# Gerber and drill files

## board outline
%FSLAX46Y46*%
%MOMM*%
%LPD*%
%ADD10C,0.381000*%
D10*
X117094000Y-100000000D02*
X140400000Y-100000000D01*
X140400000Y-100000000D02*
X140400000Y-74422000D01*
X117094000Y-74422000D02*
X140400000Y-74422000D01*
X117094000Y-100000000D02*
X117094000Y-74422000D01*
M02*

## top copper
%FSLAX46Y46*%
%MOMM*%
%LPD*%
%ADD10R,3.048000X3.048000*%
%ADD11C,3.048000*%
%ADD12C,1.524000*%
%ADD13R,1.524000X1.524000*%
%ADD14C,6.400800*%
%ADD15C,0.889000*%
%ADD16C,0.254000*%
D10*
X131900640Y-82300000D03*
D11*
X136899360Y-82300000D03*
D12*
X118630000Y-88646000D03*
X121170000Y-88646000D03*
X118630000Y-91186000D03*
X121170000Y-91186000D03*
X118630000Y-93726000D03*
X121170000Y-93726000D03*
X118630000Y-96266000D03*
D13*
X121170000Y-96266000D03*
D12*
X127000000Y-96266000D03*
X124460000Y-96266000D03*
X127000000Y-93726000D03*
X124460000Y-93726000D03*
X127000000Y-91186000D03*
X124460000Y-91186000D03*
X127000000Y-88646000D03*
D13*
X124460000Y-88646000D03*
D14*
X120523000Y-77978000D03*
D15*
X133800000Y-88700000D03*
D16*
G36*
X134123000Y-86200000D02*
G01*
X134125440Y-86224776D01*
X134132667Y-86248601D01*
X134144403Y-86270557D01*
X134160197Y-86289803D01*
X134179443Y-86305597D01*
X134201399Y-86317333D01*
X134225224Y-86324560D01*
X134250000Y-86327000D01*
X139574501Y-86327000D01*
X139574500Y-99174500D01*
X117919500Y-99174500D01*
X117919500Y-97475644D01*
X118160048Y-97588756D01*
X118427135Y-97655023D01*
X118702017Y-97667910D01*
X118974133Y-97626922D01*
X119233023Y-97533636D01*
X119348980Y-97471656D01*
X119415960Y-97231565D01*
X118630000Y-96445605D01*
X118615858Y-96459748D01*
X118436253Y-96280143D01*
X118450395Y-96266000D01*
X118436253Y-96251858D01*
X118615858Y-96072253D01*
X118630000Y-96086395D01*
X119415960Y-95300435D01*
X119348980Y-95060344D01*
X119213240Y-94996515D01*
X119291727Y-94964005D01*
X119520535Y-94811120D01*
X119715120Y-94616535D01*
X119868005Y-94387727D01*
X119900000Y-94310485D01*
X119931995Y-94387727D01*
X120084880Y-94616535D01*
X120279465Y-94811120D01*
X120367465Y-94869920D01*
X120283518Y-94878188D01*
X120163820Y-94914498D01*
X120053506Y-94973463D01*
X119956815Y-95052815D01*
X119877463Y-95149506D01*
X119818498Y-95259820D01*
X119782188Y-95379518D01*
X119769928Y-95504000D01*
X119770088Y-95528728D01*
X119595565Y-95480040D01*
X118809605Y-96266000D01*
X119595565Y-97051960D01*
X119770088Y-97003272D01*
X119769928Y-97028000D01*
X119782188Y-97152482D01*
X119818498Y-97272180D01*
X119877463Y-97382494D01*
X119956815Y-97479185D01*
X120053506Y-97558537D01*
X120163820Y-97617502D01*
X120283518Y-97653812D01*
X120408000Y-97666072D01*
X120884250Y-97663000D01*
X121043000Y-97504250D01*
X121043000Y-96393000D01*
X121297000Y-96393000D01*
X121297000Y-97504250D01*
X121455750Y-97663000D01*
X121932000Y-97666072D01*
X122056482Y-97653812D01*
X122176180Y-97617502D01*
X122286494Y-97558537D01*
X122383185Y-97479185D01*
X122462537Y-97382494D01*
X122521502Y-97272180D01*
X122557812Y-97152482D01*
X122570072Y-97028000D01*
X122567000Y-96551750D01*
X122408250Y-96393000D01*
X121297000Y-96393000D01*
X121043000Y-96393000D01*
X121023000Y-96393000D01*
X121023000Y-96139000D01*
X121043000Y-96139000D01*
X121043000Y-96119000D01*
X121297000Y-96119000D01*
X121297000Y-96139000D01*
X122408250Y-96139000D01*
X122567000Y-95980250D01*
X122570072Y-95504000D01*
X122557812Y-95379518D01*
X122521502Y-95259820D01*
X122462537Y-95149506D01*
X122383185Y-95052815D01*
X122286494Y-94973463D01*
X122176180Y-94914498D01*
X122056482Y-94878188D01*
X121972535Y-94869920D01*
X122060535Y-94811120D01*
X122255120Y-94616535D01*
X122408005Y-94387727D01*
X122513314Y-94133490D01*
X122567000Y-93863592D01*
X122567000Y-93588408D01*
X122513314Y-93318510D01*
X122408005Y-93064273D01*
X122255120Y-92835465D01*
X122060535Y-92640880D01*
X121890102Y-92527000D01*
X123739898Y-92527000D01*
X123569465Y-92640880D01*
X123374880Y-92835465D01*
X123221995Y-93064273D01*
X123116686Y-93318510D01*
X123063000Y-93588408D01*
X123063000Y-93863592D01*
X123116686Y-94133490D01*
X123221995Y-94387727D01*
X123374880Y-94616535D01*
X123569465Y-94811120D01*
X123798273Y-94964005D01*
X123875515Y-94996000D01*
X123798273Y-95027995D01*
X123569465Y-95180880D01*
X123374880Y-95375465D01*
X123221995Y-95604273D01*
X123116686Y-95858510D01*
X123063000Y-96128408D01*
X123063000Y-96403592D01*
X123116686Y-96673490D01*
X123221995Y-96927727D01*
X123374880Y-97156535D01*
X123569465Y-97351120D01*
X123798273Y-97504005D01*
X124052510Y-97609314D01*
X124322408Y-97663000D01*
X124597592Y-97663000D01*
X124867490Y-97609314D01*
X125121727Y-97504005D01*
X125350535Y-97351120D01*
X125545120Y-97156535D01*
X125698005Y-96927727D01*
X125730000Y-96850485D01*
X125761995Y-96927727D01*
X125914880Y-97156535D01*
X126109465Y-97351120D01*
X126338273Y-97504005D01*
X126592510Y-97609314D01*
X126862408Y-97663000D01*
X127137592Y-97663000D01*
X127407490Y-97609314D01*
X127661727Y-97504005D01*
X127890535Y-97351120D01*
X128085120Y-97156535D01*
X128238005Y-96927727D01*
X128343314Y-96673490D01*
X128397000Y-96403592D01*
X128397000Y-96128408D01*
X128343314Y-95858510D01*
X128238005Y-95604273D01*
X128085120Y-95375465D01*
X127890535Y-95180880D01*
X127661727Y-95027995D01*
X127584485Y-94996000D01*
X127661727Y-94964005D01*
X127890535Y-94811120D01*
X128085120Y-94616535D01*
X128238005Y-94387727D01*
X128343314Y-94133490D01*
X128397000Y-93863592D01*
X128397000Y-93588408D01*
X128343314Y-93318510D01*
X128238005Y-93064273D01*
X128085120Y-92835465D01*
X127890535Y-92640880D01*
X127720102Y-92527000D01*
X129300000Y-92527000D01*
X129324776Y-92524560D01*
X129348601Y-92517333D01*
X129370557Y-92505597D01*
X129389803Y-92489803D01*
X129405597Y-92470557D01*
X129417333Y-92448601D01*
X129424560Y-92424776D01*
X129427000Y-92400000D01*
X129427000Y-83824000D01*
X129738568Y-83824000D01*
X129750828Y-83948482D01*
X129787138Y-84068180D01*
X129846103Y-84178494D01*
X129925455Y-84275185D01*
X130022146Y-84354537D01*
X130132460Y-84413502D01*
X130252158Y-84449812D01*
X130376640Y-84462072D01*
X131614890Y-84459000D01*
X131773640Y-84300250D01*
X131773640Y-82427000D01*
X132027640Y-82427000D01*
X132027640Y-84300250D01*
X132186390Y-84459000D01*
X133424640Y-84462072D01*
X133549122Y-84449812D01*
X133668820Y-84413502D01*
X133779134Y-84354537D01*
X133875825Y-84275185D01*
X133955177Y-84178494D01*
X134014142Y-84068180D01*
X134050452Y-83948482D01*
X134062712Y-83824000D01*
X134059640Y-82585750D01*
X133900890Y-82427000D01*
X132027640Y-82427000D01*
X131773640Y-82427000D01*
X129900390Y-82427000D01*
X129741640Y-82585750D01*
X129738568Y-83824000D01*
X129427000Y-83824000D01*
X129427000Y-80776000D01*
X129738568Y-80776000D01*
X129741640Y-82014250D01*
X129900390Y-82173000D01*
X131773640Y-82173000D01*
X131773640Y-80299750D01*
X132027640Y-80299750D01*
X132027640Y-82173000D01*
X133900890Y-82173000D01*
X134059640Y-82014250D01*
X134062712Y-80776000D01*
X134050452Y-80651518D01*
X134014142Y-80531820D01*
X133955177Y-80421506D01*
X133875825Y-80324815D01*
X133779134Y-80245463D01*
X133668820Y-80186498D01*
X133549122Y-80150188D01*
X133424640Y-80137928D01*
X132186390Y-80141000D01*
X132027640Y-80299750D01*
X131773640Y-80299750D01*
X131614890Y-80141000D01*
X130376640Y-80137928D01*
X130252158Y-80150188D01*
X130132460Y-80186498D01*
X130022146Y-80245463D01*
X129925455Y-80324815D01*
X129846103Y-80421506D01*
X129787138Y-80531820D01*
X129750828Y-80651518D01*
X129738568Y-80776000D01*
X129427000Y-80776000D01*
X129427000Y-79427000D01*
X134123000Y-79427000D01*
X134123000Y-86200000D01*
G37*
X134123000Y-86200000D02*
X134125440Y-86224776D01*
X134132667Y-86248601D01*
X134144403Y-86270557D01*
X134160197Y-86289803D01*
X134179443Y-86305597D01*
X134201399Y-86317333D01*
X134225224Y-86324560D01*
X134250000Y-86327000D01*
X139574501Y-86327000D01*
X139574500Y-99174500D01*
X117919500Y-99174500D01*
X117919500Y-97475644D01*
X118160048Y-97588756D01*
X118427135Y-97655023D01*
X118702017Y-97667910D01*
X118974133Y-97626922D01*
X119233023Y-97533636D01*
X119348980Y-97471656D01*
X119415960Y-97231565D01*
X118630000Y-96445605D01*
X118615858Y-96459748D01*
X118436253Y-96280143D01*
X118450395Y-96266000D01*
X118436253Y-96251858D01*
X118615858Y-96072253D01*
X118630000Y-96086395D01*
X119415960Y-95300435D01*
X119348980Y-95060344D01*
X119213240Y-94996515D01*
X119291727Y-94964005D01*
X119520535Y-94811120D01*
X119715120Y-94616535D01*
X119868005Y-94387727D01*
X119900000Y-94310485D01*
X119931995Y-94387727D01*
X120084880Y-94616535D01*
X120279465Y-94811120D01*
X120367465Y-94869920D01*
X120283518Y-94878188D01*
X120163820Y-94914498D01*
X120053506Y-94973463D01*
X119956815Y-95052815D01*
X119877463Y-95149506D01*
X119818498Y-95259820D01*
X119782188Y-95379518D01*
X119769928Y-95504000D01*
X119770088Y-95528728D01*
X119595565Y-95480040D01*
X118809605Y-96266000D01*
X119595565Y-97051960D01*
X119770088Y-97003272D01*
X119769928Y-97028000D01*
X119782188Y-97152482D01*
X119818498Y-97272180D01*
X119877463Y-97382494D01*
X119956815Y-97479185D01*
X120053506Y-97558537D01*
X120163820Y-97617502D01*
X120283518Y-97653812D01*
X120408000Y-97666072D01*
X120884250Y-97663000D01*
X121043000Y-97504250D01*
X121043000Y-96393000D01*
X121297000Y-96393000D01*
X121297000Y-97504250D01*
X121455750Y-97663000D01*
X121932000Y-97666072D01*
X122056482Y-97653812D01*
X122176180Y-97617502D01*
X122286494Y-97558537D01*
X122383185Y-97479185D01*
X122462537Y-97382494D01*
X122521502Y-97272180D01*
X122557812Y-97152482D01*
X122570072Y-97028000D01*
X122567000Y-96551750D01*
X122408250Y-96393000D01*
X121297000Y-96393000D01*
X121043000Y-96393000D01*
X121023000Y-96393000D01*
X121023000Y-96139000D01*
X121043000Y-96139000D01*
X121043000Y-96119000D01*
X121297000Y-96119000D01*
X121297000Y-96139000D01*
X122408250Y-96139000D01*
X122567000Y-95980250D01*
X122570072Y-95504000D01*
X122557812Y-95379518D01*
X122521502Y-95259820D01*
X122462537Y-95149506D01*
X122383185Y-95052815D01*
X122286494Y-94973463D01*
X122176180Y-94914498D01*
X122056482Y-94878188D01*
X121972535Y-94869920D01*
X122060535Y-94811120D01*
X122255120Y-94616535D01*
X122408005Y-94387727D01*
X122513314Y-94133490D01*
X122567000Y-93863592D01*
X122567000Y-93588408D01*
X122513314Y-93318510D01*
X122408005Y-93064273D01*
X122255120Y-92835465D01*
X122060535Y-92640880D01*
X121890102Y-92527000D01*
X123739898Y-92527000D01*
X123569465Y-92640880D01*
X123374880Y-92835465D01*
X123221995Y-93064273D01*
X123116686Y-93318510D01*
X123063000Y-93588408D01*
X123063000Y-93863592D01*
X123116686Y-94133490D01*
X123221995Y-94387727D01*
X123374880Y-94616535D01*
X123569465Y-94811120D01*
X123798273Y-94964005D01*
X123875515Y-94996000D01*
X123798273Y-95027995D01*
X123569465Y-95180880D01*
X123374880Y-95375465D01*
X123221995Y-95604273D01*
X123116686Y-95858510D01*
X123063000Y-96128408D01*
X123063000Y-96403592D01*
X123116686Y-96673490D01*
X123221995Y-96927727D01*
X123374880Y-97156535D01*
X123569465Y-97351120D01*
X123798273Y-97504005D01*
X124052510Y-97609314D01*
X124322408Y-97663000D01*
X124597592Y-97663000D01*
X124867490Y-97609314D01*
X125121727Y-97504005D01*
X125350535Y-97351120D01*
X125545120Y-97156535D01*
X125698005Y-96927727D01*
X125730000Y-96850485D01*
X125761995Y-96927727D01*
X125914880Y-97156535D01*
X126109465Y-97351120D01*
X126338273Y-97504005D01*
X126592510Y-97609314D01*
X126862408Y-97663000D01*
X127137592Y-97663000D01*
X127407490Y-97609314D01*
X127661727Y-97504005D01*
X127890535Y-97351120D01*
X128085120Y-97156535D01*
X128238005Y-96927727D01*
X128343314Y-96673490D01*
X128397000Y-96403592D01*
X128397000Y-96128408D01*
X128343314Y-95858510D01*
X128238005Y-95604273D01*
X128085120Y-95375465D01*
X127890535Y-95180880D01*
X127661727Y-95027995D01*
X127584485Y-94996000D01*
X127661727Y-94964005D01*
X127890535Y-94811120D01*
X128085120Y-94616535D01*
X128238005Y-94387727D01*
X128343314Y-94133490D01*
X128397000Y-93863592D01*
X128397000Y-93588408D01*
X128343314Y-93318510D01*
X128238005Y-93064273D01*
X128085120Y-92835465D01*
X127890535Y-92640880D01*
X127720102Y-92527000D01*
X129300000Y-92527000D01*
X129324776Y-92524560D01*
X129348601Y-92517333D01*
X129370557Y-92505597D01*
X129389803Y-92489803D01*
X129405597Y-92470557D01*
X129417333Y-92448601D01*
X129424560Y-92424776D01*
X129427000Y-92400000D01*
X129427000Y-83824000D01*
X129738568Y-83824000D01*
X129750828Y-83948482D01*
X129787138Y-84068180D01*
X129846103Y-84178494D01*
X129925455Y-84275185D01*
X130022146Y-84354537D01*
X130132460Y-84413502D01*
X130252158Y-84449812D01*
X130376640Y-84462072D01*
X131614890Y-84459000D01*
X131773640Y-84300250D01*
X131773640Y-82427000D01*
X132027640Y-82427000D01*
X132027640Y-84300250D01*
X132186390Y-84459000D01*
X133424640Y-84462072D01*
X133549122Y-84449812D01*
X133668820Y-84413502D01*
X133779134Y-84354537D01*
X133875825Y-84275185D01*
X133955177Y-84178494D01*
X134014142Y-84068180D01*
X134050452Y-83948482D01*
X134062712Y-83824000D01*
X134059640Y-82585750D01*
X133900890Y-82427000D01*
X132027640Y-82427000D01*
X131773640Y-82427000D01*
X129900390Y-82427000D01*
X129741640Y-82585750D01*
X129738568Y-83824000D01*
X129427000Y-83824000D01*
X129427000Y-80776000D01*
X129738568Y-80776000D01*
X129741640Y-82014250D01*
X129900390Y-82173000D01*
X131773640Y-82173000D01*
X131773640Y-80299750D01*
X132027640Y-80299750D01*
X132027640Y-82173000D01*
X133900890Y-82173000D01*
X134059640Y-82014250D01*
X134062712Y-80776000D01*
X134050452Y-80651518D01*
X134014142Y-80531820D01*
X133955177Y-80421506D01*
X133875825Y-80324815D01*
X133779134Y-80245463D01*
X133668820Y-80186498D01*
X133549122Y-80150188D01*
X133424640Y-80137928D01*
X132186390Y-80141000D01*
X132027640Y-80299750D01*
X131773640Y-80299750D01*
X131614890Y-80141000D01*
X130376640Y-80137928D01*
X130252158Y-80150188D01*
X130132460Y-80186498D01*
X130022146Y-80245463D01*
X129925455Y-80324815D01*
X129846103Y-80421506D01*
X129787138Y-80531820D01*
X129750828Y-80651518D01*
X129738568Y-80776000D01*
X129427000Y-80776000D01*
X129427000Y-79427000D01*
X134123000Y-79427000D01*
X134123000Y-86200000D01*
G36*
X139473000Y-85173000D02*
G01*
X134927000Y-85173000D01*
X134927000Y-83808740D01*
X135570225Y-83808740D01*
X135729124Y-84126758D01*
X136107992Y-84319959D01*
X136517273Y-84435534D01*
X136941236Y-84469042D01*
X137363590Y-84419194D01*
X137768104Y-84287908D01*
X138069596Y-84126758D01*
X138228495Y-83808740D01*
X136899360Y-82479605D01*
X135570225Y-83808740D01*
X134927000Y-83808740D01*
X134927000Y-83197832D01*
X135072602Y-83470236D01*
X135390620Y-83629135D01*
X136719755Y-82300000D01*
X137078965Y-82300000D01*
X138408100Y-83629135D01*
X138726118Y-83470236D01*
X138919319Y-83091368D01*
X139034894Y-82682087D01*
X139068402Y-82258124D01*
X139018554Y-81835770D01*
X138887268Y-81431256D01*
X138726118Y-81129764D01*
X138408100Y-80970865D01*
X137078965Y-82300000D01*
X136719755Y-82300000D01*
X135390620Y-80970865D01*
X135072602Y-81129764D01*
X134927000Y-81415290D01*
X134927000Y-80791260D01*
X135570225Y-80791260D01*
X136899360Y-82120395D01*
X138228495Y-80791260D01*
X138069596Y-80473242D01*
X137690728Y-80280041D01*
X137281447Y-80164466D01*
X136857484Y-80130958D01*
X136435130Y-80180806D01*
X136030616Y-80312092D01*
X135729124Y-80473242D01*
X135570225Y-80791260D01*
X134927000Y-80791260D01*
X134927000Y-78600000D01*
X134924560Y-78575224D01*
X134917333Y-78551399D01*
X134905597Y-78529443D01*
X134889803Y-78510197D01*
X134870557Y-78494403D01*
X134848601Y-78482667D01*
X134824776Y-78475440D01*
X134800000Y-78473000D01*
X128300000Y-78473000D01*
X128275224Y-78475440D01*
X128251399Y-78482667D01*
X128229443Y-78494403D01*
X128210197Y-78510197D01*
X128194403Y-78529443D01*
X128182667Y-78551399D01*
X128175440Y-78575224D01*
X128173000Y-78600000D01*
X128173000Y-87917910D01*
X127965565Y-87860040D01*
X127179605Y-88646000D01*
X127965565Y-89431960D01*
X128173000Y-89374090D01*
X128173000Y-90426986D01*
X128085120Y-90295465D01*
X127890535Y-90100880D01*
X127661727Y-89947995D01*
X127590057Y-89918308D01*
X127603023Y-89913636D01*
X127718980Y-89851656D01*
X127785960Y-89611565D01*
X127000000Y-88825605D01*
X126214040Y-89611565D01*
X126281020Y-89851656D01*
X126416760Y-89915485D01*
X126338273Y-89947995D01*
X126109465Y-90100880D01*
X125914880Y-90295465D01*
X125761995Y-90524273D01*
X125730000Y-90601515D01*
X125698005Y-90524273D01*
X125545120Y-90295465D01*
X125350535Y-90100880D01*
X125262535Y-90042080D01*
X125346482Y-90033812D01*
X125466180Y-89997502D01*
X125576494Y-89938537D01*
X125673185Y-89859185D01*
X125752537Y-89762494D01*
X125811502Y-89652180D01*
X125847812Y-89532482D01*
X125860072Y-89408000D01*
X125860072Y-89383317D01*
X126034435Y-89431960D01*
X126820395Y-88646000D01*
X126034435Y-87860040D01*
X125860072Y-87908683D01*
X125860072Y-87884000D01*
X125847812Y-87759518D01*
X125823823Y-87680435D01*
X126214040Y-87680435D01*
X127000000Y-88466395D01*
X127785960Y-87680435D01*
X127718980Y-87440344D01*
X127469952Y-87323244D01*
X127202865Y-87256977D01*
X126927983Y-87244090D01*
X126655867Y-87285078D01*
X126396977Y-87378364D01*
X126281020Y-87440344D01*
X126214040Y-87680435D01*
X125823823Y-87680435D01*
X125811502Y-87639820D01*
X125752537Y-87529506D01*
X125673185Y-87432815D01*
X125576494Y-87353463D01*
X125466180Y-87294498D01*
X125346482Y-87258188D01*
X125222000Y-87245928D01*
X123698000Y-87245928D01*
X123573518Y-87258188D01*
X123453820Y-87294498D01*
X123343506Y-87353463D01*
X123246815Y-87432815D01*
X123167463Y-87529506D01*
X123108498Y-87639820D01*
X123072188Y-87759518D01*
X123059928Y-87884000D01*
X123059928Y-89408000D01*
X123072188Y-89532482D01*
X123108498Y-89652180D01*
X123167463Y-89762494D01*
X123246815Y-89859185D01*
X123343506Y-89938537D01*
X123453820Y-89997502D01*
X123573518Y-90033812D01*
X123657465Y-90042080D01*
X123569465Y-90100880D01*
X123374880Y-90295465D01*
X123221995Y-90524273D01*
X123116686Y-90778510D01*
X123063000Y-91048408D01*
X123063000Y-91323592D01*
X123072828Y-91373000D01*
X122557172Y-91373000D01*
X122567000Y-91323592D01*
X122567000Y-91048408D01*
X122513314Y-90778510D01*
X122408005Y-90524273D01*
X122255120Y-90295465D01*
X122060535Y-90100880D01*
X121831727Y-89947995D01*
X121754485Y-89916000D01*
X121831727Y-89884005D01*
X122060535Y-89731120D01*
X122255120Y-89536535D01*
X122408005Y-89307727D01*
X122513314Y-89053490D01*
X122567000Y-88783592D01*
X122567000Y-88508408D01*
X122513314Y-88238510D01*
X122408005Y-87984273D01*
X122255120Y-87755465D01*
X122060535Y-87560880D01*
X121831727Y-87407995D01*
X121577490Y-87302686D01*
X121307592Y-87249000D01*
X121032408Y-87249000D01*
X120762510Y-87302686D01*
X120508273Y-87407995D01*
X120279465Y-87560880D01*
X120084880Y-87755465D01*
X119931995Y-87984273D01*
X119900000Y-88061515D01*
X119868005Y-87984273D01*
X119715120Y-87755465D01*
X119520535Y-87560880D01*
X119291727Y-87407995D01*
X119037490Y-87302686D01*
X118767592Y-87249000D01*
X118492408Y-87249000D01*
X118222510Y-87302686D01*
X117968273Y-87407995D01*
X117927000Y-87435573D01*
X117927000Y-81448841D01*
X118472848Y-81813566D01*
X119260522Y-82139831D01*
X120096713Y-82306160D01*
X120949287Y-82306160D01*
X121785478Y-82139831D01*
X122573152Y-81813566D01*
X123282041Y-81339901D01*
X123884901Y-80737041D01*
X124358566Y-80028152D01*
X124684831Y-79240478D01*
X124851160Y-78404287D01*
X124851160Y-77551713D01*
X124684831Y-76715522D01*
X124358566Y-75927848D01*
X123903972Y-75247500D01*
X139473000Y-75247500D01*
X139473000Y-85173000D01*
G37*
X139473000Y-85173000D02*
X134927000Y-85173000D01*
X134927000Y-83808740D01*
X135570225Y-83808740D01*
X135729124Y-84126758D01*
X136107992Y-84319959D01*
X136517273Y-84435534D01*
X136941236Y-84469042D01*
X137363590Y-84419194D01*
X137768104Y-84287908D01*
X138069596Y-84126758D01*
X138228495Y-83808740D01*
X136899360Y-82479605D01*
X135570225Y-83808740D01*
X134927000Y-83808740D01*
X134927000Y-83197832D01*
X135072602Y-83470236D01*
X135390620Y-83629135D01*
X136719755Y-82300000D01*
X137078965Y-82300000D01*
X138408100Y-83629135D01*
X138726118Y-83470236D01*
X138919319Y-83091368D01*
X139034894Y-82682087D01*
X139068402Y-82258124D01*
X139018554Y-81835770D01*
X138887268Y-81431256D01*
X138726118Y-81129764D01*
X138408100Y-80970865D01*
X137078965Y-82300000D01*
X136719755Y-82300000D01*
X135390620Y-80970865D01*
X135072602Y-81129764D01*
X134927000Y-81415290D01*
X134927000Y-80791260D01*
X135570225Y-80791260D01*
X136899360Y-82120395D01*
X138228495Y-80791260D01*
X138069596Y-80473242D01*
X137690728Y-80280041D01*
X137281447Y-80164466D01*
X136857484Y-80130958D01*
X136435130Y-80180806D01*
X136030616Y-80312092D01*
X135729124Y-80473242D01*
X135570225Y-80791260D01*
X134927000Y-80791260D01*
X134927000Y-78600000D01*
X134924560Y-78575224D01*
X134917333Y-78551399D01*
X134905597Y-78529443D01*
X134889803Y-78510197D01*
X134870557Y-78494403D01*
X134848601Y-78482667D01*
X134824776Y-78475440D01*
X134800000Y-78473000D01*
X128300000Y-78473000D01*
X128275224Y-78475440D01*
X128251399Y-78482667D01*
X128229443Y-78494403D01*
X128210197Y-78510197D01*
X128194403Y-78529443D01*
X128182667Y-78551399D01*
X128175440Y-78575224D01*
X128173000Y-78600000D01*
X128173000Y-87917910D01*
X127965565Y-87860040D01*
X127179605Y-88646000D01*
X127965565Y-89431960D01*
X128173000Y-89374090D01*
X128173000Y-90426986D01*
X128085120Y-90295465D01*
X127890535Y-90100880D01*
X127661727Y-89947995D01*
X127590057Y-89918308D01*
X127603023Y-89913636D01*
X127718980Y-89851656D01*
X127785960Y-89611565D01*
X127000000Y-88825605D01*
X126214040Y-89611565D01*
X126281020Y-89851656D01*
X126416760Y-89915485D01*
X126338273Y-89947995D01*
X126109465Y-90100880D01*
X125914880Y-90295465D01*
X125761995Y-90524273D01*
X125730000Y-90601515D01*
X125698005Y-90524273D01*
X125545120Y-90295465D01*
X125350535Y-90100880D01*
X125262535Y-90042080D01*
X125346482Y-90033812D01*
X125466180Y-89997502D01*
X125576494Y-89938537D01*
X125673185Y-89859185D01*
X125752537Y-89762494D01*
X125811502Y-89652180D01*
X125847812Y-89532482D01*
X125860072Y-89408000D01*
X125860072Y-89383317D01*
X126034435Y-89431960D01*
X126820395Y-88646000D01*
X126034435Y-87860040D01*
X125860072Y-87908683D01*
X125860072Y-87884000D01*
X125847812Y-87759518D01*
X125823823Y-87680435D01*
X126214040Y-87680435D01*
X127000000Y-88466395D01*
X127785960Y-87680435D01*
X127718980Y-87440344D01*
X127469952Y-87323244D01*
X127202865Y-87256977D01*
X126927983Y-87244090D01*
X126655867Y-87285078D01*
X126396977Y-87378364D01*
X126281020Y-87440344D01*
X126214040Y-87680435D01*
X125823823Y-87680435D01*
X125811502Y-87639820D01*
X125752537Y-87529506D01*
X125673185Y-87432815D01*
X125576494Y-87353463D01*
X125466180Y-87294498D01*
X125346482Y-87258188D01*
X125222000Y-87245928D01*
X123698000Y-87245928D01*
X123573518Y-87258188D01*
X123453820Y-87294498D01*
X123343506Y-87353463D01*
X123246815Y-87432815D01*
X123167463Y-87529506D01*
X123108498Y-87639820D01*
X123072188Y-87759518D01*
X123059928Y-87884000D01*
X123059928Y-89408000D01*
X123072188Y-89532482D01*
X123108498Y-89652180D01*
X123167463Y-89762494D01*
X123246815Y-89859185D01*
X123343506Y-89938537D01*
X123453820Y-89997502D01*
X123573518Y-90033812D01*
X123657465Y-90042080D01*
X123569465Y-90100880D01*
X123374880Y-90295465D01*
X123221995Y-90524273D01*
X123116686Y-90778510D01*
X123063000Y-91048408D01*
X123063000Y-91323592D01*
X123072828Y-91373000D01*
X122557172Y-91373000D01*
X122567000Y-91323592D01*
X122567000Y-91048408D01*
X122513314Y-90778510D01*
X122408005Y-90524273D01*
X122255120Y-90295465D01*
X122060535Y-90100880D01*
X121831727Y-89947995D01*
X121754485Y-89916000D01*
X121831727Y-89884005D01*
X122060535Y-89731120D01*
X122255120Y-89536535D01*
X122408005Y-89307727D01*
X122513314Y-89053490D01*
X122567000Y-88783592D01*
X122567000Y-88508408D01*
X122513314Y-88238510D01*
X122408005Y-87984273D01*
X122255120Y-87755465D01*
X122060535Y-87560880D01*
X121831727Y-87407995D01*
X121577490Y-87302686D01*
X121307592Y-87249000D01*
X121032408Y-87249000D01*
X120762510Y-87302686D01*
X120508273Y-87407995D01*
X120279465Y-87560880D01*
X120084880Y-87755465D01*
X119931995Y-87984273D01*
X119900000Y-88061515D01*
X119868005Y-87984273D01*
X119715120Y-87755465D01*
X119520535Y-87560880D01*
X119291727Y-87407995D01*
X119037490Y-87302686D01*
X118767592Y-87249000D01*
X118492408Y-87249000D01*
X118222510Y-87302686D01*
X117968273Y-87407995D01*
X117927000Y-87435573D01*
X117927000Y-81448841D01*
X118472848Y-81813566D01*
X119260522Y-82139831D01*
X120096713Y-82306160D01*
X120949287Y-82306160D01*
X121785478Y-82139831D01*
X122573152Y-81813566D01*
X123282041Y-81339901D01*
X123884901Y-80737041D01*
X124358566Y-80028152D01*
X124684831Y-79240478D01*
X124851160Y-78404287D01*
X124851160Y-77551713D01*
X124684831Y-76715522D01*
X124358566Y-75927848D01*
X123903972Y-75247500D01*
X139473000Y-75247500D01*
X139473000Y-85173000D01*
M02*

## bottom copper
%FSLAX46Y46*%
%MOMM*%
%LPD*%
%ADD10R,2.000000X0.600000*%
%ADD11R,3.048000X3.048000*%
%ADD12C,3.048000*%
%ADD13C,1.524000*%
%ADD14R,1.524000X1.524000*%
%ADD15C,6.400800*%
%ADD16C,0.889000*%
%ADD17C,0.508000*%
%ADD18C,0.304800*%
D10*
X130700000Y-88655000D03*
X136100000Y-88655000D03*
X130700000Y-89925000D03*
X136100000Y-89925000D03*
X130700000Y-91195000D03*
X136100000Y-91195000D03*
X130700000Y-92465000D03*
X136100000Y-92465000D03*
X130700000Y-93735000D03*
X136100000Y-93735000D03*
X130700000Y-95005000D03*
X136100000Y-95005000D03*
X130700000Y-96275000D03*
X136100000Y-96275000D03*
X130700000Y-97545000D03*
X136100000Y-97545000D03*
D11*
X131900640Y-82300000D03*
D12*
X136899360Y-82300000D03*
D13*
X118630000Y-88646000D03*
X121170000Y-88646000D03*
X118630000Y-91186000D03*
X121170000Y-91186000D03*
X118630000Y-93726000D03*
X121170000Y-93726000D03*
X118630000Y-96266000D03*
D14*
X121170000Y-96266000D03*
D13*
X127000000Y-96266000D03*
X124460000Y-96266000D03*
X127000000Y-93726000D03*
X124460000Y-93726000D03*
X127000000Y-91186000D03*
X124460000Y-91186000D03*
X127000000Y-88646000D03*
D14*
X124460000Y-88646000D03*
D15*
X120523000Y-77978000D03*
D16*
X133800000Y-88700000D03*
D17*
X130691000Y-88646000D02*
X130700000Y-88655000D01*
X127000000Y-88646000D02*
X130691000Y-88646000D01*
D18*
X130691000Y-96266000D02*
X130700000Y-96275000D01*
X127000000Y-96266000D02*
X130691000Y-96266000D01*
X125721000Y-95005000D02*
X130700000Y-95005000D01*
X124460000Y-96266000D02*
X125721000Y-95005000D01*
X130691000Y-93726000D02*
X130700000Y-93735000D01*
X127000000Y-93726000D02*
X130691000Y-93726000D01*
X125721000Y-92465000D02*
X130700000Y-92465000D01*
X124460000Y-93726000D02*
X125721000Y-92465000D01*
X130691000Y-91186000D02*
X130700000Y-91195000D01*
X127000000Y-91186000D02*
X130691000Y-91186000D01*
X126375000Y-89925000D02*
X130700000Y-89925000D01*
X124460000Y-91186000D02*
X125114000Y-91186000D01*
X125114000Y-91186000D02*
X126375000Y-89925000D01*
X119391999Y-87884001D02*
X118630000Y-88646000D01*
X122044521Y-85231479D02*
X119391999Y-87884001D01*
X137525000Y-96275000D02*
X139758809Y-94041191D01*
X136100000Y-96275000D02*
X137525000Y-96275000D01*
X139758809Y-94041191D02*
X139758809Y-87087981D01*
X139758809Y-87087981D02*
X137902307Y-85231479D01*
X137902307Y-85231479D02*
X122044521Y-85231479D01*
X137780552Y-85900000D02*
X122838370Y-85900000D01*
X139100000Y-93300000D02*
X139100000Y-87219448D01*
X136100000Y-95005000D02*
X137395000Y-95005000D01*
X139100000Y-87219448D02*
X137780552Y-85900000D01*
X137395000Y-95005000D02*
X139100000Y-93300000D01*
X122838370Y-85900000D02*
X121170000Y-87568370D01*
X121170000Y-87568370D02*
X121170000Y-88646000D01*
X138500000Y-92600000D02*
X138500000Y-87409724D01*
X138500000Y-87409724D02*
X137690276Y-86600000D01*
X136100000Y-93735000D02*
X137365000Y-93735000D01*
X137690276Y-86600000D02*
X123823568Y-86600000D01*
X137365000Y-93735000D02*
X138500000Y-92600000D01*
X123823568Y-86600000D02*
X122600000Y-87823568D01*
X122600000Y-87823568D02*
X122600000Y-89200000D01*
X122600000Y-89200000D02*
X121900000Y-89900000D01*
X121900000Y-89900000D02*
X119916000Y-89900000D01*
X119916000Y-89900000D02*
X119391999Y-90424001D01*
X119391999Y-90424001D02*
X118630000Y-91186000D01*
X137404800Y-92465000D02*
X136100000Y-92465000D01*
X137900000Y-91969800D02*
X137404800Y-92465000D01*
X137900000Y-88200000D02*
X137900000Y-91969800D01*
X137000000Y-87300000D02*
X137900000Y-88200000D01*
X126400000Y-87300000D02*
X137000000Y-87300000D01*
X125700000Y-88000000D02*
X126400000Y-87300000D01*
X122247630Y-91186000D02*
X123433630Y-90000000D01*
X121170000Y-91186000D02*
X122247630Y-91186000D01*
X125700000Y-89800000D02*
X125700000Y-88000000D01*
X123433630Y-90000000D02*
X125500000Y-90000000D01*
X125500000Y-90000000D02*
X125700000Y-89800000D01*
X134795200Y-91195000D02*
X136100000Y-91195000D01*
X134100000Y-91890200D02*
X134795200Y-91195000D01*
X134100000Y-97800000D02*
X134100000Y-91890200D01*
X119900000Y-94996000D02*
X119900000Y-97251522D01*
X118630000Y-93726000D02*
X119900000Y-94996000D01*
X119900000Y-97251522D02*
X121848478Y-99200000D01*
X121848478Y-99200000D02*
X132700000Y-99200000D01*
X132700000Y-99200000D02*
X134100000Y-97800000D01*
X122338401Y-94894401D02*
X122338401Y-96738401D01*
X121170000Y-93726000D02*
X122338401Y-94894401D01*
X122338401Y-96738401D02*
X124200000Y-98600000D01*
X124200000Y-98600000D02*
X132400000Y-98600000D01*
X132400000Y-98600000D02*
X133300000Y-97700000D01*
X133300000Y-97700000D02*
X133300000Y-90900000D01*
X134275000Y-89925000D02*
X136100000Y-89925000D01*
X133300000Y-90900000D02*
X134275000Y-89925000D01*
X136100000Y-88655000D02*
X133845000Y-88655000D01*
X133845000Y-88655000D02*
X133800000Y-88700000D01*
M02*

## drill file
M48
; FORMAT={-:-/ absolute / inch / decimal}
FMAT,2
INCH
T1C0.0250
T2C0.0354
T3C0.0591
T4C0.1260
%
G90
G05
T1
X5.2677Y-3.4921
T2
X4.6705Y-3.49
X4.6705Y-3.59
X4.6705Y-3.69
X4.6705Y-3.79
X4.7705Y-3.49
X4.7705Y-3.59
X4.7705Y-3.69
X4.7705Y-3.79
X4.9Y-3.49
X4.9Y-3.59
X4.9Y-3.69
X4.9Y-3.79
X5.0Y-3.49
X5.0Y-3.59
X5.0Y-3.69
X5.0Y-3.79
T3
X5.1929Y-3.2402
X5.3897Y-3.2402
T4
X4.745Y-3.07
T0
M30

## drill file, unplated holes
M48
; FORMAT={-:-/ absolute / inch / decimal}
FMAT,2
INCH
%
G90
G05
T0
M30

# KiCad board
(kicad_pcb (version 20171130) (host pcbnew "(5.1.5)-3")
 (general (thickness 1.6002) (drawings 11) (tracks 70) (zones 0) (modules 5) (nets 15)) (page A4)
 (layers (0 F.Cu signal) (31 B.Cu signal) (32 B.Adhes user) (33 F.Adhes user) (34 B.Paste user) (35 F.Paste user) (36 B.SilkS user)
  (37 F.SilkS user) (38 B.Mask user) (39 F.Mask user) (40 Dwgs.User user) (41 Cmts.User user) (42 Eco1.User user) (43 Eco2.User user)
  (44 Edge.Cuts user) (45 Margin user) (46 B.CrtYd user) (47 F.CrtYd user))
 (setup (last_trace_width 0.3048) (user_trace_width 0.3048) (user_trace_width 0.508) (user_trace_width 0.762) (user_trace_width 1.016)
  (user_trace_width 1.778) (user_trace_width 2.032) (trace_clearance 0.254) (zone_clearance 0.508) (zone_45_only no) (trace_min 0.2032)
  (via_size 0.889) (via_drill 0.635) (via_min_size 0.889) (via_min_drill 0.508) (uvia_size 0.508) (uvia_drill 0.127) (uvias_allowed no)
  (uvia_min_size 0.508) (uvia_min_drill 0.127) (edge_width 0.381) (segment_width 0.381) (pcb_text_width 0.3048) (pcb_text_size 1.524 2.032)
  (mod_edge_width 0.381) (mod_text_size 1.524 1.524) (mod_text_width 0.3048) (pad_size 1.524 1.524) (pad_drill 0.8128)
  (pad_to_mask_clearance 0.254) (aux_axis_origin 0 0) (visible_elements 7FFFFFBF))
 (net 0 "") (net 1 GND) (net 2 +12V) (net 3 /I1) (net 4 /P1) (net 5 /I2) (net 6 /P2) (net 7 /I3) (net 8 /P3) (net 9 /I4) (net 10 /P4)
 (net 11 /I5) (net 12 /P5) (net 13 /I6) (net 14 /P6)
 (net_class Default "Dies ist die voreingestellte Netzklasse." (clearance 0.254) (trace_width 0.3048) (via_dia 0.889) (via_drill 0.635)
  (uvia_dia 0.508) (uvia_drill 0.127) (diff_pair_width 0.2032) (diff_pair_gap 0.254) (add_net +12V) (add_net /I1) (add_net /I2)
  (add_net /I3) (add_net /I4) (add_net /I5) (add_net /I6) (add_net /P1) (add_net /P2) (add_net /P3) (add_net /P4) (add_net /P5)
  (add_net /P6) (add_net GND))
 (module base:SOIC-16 (layer B.Cu) (at 133.4 93.1 90)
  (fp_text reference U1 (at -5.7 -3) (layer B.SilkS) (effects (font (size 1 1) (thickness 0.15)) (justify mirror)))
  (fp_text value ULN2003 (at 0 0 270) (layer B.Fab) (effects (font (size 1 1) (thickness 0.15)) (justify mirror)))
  (pad 8 smd rect (at 4.445 -2.7 90) (size 0.6 2) (layers B.Cu B.Paste B.Mask) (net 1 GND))
  (pad 9 smd rect (at 4.445 2.7 90) (size 0.6 2) (layers B.Cu B.Paste B.Mask) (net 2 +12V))
  (pad 7 smd rect (at 3.175 -2.7 90) (size 0.6 2) (layers B.Cu B.Paste B.Mask) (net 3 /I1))
  (pad 10 smd rect (at 3.175 2.7 90) (size 0.6 2) (layers B.Cu B.Paste B.Mask) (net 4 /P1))
  (pad 6 smd rect (at 1.905 -2.7 90) (size 0.6 2) (layers B.Cu B.Paste B.Mask) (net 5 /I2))
  (pad 11 smd rect (at 1.905 2.7 90) (size 0.6 2) (layers B.Cu B.Paste B.Mask) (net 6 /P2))
  (pad 5 smd rect (at 0.635 -2.7 90) (size 0.6 2) (layers B.Cu B.Paste B.Mask) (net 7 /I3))
  (pad 12 smd rect (at 0.635 2.7 90) (size 0.6 2) (layers B.Cu B.Paste B.Mask) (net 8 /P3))
  (pad 4 smd rect (at -0.635 -2.7 90) (size 0.6 2) (layers B.Cu B.Paste B.Mask) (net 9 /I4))
  (pad 13 smd rect (at -0.635 2.7 90) (size 0.6 2) (layers B.Cu B.Paste B.Mask) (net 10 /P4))
  (pad 3 smd rect (at -1.905 -2.7 90) (size 0.6 2) (layers B.Cu B.Paste B.Mask) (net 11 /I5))
  (pad 14 smd rect (at -1.905 2.7 90) (size 0.6 2) (layers B.Cu B.Paste B.Mask) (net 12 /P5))
  (pad 2 smd rect (at -3.175 -2.7 90) (size 0.6 2) (layers B.Cu B.Paste B.Mask) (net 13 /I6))
  (pad 15 smd rect (at -3.175 2.7 90) (size 0.6 2) (layers B.Cu B.Paste B.Mask) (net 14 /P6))
  (pad 1 smd rect (at -4.445 -2.7 90) (size 0.6 2) (layers B.Cu B.Paste B.Mask))
  (pad 16 smd rect (at -4.445 2.7 90) (size 0.6 2) (layers B.Cu B.Paste B.Mask)))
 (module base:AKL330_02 (layer F.Cu) (at 134.4 82.3)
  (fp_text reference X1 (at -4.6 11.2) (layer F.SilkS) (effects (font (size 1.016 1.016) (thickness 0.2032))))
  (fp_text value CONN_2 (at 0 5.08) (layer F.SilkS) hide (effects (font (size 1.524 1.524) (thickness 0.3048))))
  (pad 1 thru_hole rect (at -2.49936 0) (size 3.048 3.048) (drill 1.50114) (layers *.Cu *.Mask F.SilkS) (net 2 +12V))
  (pad 2 thru_hole circle (at 2.49936 0) (size 3.048 3.048) (drill 1.50114) (layers *.Cu *.Mask F.SilkS) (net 1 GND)))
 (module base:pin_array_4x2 (layer F.Cu) (at 119.9 92.456 90)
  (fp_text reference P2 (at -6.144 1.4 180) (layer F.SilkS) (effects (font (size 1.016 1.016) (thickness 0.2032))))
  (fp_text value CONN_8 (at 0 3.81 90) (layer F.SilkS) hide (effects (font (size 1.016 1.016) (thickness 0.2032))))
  (pad 8 thru_hole circle (at 3.81 -1.27 90) (size 1.524 1.524) (drill 0.89916) (layers *.Cu *.Mask F.SilkS) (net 14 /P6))
  (pad 7 thru_hole circle (at 3.81 1.27 90) (size 1.524 1.524) (drill 0.89916) (layers *.Cu *.Mask F.SilkS) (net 12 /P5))
  (pad 6 thru_hole circle (at 1.27 -1.27 90) (size 1.524 1.524) (drill 0.89916) (layers *.Cu *.Mask F.SilkS) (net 10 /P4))
  (pad 5 thru_hole circle (at 1.27 1.27 90) (size 1.524 1.524) (drill 0.89916) (layers *.Cu *.Mask F.SilkS) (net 8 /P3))
  (pad 4 thru_hole circle (at -1.27 -1.27 90) (size 1.524 1.524) (drill 0.89916) (layers *.Cu *.Mask F.SilkS) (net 6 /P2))
  (pad 3 thru_hole circle (at -1.27 1.27 90) (size 1.524 1.524) (drill 0.89916) (layers *.Cu *.Mask F.SilkS) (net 4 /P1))
  (pad 2 thru_hole circle (at -3.81 -1.27 90) (size 1.524 1.524) (drill 0.89916) (layers *.Cu *.Mask F.SilkS) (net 2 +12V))
  (pad 1 thru_hole rect (at -3.81 1.27 90) (size 1.524 1.524) (drill 0.89916) (layers *.Cu *.Mask F.SilkS) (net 2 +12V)))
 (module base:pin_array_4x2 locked (layer F.Cu) (at 125.73 92.456 270)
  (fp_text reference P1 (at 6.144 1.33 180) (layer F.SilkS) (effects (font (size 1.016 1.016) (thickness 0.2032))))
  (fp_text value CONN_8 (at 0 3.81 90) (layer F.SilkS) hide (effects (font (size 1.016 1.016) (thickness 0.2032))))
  (pad 8 thru_hole circle (at 3.81 -1.27 270) (size 1.524 1.524) (drill 0.89916) (layers *.Cu *.Mask F.SilkS) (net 13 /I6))
  (pad 7 thru_hole circle (at 3.81 1.27 270) (size 1.524 1.524) (drill 0.89916) (layers *.Cu *.Mask F.SilkS) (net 11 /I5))
  (pad 6 thru_hole circle (at 1.27 -1.27 270) (size 1.524 1.524) (drill 0.89916) (layers *.Cu *.Mask F.SilkS) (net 9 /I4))
  (pad 5 thru_hole circle (at 1.27 1.27 270) (size 1.524 1.524) (drill 0.89916) (layers *.Cu *.Mask F.SilkS) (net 7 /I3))
  (pad 4 thru_hole circle (at -1.27 -1.27 270) (size 1.524 1.524) (drill 0.89916) (layers *.Cu *.Mask F.SilkS) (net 5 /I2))
  (pad 3 thru_hole circle (at -1.27 1.27 270) (size 1.524 1.524) (drill 0.89916) (layers *.Cu *.Mask F.SilkS) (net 3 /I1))
  (pad 2 thru_hole circle (at -3.81 -1.27 270) (size 1.524 1.524) (drill 0.89916) (layers *.Cu *.Mask F.SilkS) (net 1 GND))
  (pad 1 thru_hole rect (at -3.81 1.27 270) (size 1.524 1.524) (drill 0.89916) (layers *.Cu *.Mask F.SilkS)))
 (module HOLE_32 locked (layer F.Cu) (at 120.523 77.978)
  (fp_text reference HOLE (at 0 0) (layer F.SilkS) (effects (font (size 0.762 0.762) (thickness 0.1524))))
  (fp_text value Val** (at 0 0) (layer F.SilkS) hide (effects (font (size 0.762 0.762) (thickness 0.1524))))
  (pad "" thru_hole circle (at 0 0) (size 6.4008 6.4008) (drill 3.2004) (layers *.Cu *.Mask F.SilkS) (clearance 1.00076)))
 (gr_line (start 117.094 100) (end 140.4 100) (angle 90) (layer Edge.Cuts) (width 0.381))
 (gr_line (start 140.4 100) (end 140.4 74.422) (angle 90) (layer Edge.Cuts) (width 0.381))
 (gr_line (start 117.094 74.422) (end 140.4 74.422) (angle 90) (layer Edge.Cuts) (width 0.381))
 (gr_line (start 117.094 100) (end 117.094 74.422) (angle 90) (layer Edge.Cuts) (width 0.381))
 (segment (start 130.691 88.646) (end 130.7 88.655) (width 0.508) (layer B.Cu) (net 1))
 (segment (start 127 88.646) (end 130.691 88.646) (width 0.508) (layer B.Cu) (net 1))
 (segment (start 130.691 96.266) (end 130.7 96.275) (width 0.3048) (layer B.Cu) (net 13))
 (segment (start 127 96.266) (end 130.691 96.266) (width 0.3048) (layer B.Cu) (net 13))
 (segment (start 125.721 95.005) (end 130.7 95.005) (width 0.3048) (layer B.Cu) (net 11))
 (segment (start 124.46 96.266) (end 125.721 95.005) (width 0.3048) (layer B.Cu) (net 11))
 (segment (start 130.691 93.726) (end 130.7 93.735) (width 0.3048) (layer B.Cu) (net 9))
 (segment (start 127 93.726) (end 130.691 93.726) (width 0.3048) (layer B.Cu) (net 9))
 (segment (start 125.721 92.465) (end 130.7 92.465) (width 0.3048) (layer B.Cu) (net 7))
 (segment (start 124.46 93.726) (end 125.721 92.465) (width 0.3048) (layer B.Cu) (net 7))
 (segment (start 130.691 91.186) (end 130.7 91.195) (width 0.3048) (layer B.Cu) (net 5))
 (segment (start 127 91.186) (end 130.691 91.186) (width 0.3048) (layer B.Cu) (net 5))
 (segment (start 126.375 89.925) (end 130.7 89.925) (width 0.3048) (layer B.Cu) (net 3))
 (segment (start 124.46 91.186) (end 125.114 91.186) (width 0.3048) (layer B.Cu) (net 3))
 (segment (start 125.114 91.186) (end 126.375 89.925) (width 0.3048) (layer B.Cu) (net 3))
 (segment (start 119.391999 87.884001) (end 118.63 88.646) (width 0.3048) (layer B.Cu) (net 14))
 (segment (start 122.044521 85.231479) (end 119.391999 87.884001) (width 0.3048) (layer B.Cu) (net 14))
 (segment (start 137.525 96.275) (end 139.758809 94.041191) (width 0.3048) (layer B.Cu) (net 14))
 (segment (start 136.1 96.275) (end 137.525 96.275) (width 0.3048) (layer B.Cu) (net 14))
 (segment (start 139.758809 94.041191) (end 139.758809 87.087981) (width 0.3048) (layer B.Cu) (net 14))
 (segment (start 139.758809 87.087981) (end 137.902307 85.231479) (width 0.3048) (layer B.Cu) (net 14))
 (segment (start 137.902307 85.231479) (end 122.044521 85.231479) (width 0.3048) (layer B.Cu) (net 14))
 (segment (start 137.780552 85.9) (end 122.83837 85.9) (width 0.3048) (layer B.Cu) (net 12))
 (segment (start 139.1 93.3) (end 139.1 87.219448) (width 0.3048) (layer B.Cu) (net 12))
 (segment (start 136.1 95.005) (end 137.395 95.005) (width 0.3048) (layer B.Cu) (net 12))
 (segment (start 139.1 87.219448) (end 137.780552 85.9) (width 0.3048) (layer B.Cu) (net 12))
 (segment (start 137.395 95.005) (end 139.1 93.3) (width 0.3048) (layer B.Cu) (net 12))
 (segment (start 122.83837 85.9) (end 121.17 87.56837) (width 0.3048) (layer B.Cu) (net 12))
 (segment (start 121.17 87.56837) (end 121.17 88.646) (width 0.3048) (layer B.Cu) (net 12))
 (segment (start 138.5 92.6) (end 138.5 87.409724) (width 0.3048) (layer B.Cu) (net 10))
 (segment (start 138.5 87.409724) (end 137.690276 86.6) (width 0.3048) (layer B.Cu) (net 10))
 (segment (start 136.1 93.735) (end 137.365 93.735) (width 0.3048) (layer B.Cu) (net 10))
 (segment (start 137.690276 86.6) (end 123.823568 86.6) (width 0.3048) (layer B.Cu) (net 10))
 (segment (start 137.365 93.735) (end 138.5 92.6) (width 0.3048) (layer B.Cu) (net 10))
 (segment (start 123.823568 86.6) (end 122.6 87.823568) (width 0.3048) (layer B.Cu) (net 10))
 (segment (start 122.6 87.823568) (end 122.6 89.2) (width 0.3048) (layer B.Cu) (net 10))
 (segment (start 122.6 89.2) (end 121.9 89.9) (width 0.3048) (layer B.Cu) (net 10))
 (segment (start 121.9 89.9) (end 119.916 89.9) (width 0.3048) (layer B.Cu) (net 10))
 (segment (start 119.916 89.9) (end 119.391999 90.424001) (width 0.3048) (layer B.Cu) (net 10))
 (segment (start 119.391999 90.424001) (end 118.63 91.186) (width 0.3048) (layer B.Cu) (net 10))
 (segment (start 137.4048 92.465) (end 136.1 92.465) (width 0.3048) (layer B.Cu) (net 8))
 (segment (start 137.9 91.9698) (end 137.4048 92.465) (width 0.3048) (layer B.Cu) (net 8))
 (segment (start 137.9 88.2) (end 137.9 91.9698) (width 0.3048) (layer B.Cu) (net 8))
 (segment (start 137 87.3) (end 137.9 88.2) (width 0.3048) (layer B.Cu) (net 8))
 (segment (start 126.4 87.3) (end 137 87.3) (width 0.3048) (layer B.Cu) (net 8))
 (segment (start 125.7 88) (end 126.4 87.3) (width 0.3048) (layer B.Cu) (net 8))
 (segment (start 122.24763 91.186) (end 123.43363 90) (width 0.3048) (layer B.Cu) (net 8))
 (segment (start 121.17 91.186) (end 122.24763 91.186) (width 0.3048) (layer B.Cu) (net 8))
 (segment (start 125.7 89.8) (end 125.7 88) (width 0.3048) (layer B.Cu) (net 8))
 (segment (start 123.43363 90) (end 125.5 90) (width 0.3048) (layer B.Cu) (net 8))
 (segment (start 125.5 90) (end 125.7 89.8) (width 0.3048) (layer B.Cu) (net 8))
 (segment (start 134.7952 91.195) (end 136.1 91.195) (width 0.3048) (layer B.Cu) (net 6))
 (segment (start 134.1 91.8902) (end 134.7952 91.195) (width 0.3048) (layer B.Cu) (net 6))
 (segment (start 134.1 97.8) (end 134.1 91.8902) (width 0.3048) (layer B.Cu) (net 6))
 (segment (start 119.9 94.996) (end 119.9 97.251522) (width 0.3048) (layer B.Cu) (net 6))
 (segment (start 118.63 93.726) (end 119.9 94.996) (width 0.3048) (layer B.Cu) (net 6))
 (segment (start 119.9 97.251522) (end 121.848478 99.2) (width 0.3048) (layer B.Cu) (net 6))
 (segment (start 121.848478 99.2) (end 132.7 99.2) (width 0.3048) (layer B.Cu) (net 6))
 (segment (start 132.7 99.2) (end 134.1 97.8) (width 0.3048) (layer B.Cu) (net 6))
 (segment (start 122.338401 94.894401) (end 122.338401 96.738401) (width 0.3048) (layer B.Cu) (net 4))
 (segment (start 121.17 93.726) (end 122.338401 94.894401) (width 0.3048) (layer B.Cu) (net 4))
 (segment (start 122.338401 96.738401) (end 124.2 98.6) (width 0.3048) (layer B.Cu) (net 4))
 (segment (start 124.2 98.6) (end 132.4 98.6) (width 0.3048) (layer B.Cu) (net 4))
 (segment (start 132.4 98.6) (end 133.3 97.7) (width 0.3048) (layer B.Cu) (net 4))
 (segment (start 133.3 97.7) (end 133.3 90.9) (width 0.3048) (layer B.Cu) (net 4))
 (segment (start 134.275 89.925) (end 136.1 89.925) (width 0.3048) (layer B.Cu) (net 4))
 (segment (start 133.3 90.9) (end 134.275 89.925) (width 0.3048) (layer B.Cu) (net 4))
 (segment (start 136.1 88.655) (end 133.845 88.655) (width 0.3048) (layer B.Cu) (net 2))
 (via (at 133.8 88.7) (size 0.889) (drill 0.635) (layers F.Cu B.Cu) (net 2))
 (segment (start 133.845 88.655) (end 133.8 88.7) (width 0.3048) (layer B.Cu) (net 2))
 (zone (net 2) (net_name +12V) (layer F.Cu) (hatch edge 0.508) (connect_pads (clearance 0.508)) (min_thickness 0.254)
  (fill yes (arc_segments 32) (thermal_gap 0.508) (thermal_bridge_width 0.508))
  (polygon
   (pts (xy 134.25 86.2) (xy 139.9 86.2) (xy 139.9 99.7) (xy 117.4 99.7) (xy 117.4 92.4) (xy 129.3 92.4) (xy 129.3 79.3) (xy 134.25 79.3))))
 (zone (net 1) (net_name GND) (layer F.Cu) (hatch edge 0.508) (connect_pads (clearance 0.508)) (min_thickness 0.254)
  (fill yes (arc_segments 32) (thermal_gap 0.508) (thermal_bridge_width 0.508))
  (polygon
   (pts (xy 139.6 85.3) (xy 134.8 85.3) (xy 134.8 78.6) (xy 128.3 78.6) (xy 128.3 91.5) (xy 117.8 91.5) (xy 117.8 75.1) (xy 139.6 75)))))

